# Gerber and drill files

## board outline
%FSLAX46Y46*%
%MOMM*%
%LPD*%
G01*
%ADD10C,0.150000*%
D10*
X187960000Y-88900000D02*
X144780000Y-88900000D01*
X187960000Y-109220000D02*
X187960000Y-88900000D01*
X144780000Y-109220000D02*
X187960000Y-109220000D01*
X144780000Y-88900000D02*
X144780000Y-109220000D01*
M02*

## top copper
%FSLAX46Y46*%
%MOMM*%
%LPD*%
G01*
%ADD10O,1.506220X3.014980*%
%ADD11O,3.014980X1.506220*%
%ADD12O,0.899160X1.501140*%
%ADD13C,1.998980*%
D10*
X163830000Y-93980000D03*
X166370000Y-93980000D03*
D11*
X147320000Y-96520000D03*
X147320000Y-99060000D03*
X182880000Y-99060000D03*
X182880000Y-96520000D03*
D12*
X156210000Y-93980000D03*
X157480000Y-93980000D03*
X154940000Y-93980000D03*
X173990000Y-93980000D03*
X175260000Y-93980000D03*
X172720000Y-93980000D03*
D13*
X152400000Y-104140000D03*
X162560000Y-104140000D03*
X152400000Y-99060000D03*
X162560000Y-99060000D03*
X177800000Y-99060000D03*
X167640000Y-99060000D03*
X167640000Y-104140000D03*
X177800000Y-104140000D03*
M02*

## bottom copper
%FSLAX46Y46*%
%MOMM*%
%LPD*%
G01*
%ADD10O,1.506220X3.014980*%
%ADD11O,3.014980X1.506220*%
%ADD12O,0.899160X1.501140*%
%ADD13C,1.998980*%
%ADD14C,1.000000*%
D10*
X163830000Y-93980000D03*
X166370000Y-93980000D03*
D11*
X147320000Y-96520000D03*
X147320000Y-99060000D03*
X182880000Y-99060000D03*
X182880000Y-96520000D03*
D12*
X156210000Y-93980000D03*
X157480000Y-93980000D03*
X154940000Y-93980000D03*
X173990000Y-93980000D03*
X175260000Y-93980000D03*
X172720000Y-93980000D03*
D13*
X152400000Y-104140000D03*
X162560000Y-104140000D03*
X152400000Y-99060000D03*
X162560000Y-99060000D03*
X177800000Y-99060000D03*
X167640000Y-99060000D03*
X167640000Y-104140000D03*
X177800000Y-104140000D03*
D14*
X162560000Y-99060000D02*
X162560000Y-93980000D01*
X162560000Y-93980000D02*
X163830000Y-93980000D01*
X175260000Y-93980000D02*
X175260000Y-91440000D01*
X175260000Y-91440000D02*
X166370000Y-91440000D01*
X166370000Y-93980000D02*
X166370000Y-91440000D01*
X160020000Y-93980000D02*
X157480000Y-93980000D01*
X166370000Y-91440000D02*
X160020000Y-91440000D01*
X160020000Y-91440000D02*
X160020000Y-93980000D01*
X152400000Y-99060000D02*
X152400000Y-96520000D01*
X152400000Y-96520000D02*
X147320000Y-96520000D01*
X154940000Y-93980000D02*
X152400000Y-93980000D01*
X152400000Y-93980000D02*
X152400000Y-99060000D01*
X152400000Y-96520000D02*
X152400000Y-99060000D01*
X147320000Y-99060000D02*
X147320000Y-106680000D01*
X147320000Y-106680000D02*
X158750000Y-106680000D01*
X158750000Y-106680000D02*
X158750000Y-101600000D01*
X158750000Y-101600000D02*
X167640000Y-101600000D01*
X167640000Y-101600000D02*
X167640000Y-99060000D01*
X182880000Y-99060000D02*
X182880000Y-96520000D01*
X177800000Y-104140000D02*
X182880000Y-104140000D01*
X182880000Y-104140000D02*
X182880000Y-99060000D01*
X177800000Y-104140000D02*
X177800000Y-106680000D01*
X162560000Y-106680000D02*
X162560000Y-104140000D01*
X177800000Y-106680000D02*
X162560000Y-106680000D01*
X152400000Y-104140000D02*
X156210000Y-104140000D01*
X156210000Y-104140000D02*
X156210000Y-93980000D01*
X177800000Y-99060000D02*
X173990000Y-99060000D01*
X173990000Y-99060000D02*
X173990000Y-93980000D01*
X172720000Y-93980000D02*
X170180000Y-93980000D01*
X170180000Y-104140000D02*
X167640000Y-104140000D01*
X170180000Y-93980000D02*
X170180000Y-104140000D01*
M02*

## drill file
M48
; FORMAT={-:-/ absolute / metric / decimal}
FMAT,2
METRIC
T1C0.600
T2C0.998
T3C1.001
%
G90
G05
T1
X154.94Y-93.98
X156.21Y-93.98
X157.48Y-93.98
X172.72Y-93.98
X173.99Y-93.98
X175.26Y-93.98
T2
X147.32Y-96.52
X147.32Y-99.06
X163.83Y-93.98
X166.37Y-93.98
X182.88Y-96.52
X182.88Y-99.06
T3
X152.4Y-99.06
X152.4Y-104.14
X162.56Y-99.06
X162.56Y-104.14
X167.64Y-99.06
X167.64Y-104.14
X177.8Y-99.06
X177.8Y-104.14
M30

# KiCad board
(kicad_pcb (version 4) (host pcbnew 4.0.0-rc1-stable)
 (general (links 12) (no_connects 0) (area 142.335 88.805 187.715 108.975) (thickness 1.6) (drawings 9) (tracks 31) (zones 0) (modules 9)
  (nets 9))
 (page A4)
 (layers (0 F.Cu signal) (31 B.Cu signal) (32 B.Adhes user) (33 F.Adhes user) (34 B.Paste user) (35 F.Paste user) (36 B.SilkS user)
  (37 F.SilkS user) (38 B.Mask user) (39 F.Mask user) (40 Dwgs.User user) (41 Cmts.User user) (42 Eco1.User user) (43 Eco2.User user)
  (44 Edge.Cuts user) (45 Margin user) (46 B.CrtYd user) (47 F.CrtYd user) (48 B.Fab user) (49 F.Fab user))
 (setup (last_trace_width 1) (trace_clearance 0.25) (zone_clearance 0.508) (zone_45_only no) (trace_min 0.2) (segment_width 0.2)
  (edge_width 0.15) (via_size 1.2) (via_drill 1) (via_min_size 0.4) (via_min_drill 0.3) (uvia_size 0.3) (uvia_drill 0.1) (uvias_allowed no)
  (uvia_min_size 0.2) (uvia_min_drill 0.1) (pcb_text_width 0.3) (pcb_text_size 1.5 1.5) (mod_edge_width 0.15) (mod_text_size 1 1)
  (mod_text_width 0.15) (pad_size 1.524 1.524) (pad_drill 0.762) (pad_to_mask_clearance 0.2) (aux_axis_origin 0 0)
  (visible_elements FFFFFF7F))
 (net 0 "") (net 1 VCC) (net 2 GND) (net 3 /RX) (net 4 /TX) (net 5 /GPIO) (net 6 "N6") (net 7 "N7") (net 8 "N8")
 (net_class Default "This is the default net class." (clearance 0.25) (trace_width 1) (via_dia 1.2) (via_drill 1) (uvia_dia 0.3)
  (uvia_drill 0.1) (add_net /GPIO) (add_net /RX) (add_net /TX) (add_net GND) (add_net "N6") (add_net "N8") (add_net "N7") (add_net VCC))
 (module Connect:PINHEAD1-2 (layer F.Cu) (at 165.1 93.98)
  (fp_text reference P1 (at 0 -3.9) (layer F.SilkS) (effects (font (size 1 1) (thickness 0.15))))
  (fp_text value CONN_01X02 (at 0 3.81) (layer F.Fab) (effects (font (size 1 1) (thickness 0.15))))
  (pad 1 thru_hole oval (at -1.27 0) (size 1.50622 3.01498) (drill 0.99822) (layers *.Cu *.Mask) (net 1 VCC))
  (pad 2 thru_hole oval (at 1.27 0) (size 1.50622 3.01498) (drill 0.99822) (layers *.Cu *.Mask) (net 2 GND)))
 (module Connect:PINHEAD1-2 (layer F.Cu) (at 147.32 97.79 270)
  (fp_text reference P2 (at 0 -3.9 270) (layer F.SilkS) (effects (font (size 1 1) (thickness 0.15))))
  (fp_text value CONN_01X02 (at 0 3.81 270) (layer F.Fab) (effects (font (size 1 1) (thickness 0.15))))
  (pad 1 thru_hole oval (at -1.27 0 270) (size 1.50622 3.01498) (drill 0.99822) (layers *.Cu *.Mask) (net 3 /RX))
  (pad 2 thru_hole oval (at 1.27 0 270) (size 1.50622 3.01498) (drill 0.99822) (layers *.Cu *.Mask) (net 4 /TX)))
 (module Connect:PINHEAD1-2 (layer F.Cu) (at 182.88 97.79 90)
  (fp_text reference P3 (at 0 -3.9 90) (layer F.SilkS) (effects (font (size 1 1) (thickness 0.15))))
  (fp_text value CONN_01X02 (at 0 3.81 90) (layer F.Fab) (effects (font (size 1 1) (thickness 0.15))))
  (pad 1 thru_hole oval (at -1.27 0 90) (size 1.50622 3.01498) (drill 0.99822) (layers *.Cu *.Mask) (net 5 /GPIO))
  (pad 2 thru_hole oval (at 1.27 0 90) (size 1.50622 3.01498) (drill 0.99822) (layers *.Cu *.Mask) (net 5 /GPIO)))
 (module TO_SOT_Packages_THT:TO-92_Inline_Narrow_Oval (layer F.Cu) (at 154.94 93.98)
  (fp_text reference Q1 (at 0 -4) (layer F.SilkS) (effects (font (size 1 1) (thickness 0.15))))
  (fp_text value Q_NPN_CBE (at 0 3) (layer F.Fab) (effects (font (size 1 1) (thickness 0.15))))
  (pad 2 thru_hole oval (at 1.27 0 180) (size 0.89916 1.50114) (drill 0.6) (layers *.Cu *.Mask F.SilkS) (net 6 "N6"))
  (pad 3 thru_hole oval (at 2.54 0 180) (size 0.89916 1.50114) (drill 0.6) (layers *.Cu *.Mask F.SilkS) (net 2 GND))
  (pad 1 thru_hole oval (at 0 0 180) (size 0.89916 1.50114) (drill 0.6) (layers *.Cu *.Mask F.SilkS) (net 3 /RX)))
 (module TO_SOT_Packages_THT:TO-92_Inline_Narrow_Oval (layer F.Cu) (at 172.72 93.98)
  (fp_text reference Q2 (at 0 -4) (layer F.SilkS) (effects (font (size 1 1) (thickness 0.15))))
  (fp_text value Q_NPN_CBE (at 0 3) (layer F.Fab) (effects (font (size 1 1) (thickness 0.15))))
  (pad 2 thru_hole oval (at 1.27 0 180) (size 0.89916 1.50114) (drill 0.6) (layers *.Cu *.Mask F.SilkS) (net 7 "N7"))
  (pad 3 thru_hole oval (at 2.54 0 180) (size 0.89916 1.50114) (drill 0.6) (layers *.Cu *.Mask F.SilkS) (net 2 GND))
  (pad 1 thru_hole oval (at 0 0 180) (size 0.89916 1.50114) (drill 0.6) (layers *.Cu *.Mask F.SilkS) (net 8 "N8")))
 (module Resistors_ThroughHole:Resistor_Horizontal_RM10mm (layer F.Cu) (at 157.48 104.14)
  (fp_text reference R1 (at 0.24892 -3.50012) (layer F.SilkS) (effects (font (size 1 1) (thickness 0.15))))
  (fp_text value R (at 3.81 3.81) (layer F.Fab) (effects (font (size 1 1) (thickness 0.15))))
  (pad 1 thru_hole circle (at -5.08 0) (size 1.99898 1.99898) (drill 1.00076) (layers *.Cu *.SilkS *.Mask) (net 6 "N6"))
  (pad 2 thru_hole circle (at 5.08 0) (size 1.99898 1.99898) (drill 1.00076) (layers *.Cu *.SilkS *.Mask) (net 5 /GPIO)))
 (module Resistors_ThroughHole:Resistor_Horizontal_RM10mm (layer F.Cu) (at 157.48 99.06)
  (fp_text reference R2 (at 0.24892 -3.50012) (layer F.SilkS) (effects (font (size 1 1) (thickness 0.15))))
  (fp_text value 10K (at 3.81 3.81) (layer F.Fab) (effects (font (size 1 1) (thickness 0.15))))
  (pad 1 thru_hole circle (at -5.08 0) (size 1.99898 1.99898) (drill 1.00076) (layers *.Cu *.SilkS *.Mask) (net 3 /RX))
  (pad 2 thru_hole circle (at 5.08 0) (size 1.99898 1.99898) (drill 1.00076) (layers *.Cu *.SilkS *.Mask) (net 1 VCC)))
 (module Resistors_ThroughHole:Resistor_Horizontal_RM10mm (layer F.Cu) (at 172.72 99.06 180)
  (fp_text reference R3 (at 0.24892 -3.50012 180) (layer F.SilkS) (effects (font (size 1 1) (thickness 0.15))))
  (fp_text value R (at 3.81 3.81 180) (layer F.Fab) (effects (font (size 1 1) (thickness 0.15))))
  (pad 1 thru_hole circle (at -5.08 0 180) (size 1.99898 1.99898) (drill 1.00076) (layers *.Cu *.SilkS *.Mask) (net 7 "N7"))
  (pad 2 thru_hole circle (at 5.08 0 180) (size 1.99898 1.99898) (drill 1.00076) (layers *.Cu *.SilkS *.Mask) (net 4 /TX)))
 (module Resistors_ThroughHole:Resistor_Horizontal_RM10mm (layer F.Cu) (at 172.72 104.14)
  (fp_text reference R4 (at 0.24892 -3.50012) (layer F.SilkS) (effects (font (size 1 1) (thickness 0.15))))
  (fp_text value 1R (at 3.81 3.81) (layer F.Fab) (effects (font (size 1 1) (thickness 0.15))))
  (pad 1 thru_hole circle (at -5.08 0) (size 1.99898 1.99898) (drill 1.00076) (layers *.Cu *.SilkS *.Mask) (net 8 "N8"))
  (pad 2 thru_hole circle (at 5.08 0) (size 1.99898 1.99898) (drill 1.00076) (layers *.Cu *.SilkS *.Mask) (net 5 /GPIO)))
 (gr_line (start 187.96 88.9) (end 144.78 88.9) (angle 90) (layer Edge.Cuts) (width 0.15))
 (gr_line (start 187.96 109.22) (end 187.96 88.9) (angle 90) (layer Edge.Cuts) (width 0.15))
 (gr_line (start 144.78 109.22) (end 187.96 109.22) (angle 90) (layer Edge.Cuts) (width 0.15))
 (gr_line (start 144.78 88.9) (end 144.78 109.22) (angle 90) (layer Edge.Cuts) (width 0.15))
 (segment (start 162.56 99.06) (end 162.56 93.98) (width 1) (layer B.Cu) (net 1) (status 400000))
 (segment (start 162.56 93.98) (end 163.83 93.98) (width 1) (layer B.Cu) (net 1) (status 800000))
 (segment (start 175.26 93.98) (end 175.26 91.44) (width 1) (layer B.Cu) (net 2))
 (segment (start 175.26 91.44) (end 166.37 91.44) (width 1) (layer B.Cu) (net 2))
 (segment (start 166.37 93.98) (end 166.37 91.44) (width 1) (layer B.Cu) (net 2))
 (segment (start 160.02 93.98) (end 157.48 93.98) (width 1) (layer B.Cu) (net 2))
 (segment (start 166.37 91.44) (end 160.02 91.44) (width 1) (layer B.Cu) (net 2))
 (segment (start 160.02 91.44) (end 160.02 93.98) (width 1) (layer B.Cu) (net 2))
 (segment (start 152.4 99.06) (end 152.4 96.52) (width 1) (layer B.Cu) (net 3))
 (segment (start 152.4 96.52) (end 147.32 96.52) (width 1) (layer B.Cu) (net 3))
 (segment (start 154.94 93.98) (end 152.4 93.98) (width 1) (layer B.Cu) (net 3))
 (segment (start 152.4 93.98) (end 152.4 99.06) (width 1) (layer B.Cu) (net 3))
 (segment (start 152.4 96.52) (end 152.4 99.06) (width 1) (layer B.Cu) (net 3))
 (segment (start 147.32 99.06) (end 147.32 106.68) (width 1) (layer B.Cu) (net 4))
 (segment (start 147.32 106.68) (end 158.75 106.68) (width 1) (layer B.Cu) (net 4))
 (segment (start 158.75 106.68) (end 158.75 101.6) (width 1) (layer B.Cu) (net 4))
 (segment (start 158.75 101.6) (end 167.64 101.6) (width 1) (layer B.Cu) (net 4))
 (segment (start 167.64 101.6) (end 167.64 99.06) (width 1) (layer B.Cu) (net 4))
 (segment (start 182.88 99.06) (end 182.88 96.52) (width 1) (layer B.Cu) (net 5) (status C00000))
 (segment (start 177.8 104.14) (end 182.88 104.14) (width 1) (layer B.Cu) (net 5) (status 400000))
 (segment (start 182.88 104.14) (end 182.88 99.06) (width 1) (layer B.Cu) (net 5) (status 800000))
 (segment (start 177.8 104.14) (end 177.8 106.68) (width 1) (layer B.Cu) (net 5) (status 400000))
 (segment (start 162.56 106.68) (end 162.56 104.14) (width 1) (layer B.Cu) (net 5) (status 800000))
 (segment (start 177.8 106.68) (end 162.56 106.68) (width 1) (layer B.Cu) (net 5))
 (segment (start 152.4 104.14) (end 156.21 104.14) (width 1) (layer B.Cu) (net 6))
 (segment (start 156.21 104.14) (end 156.21 93.98) (width 1) (layer B.Cu) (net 6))
 (segment (start 177.8 99.06) (end 173.99 99.06) (width 1) (layer B.Cu) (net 7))
 (segment (start 173.99 99.06) (end 173.99 93.98) (width 1) (layer B.Cu) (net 7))
 (segment (start 172.72 93.98) (end 170.18 93.98) (width 1) (layer B.Cu) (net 8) (status 400000))
 (segment (start 170.18 104.14) (end 167.64 104.14) (width 1) (layer B.Cu) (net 8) (status 800000))
 (segment (start 170.18 93.98) (end 170.18 104.14) (width 1) (layer B.Cu) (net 8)))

